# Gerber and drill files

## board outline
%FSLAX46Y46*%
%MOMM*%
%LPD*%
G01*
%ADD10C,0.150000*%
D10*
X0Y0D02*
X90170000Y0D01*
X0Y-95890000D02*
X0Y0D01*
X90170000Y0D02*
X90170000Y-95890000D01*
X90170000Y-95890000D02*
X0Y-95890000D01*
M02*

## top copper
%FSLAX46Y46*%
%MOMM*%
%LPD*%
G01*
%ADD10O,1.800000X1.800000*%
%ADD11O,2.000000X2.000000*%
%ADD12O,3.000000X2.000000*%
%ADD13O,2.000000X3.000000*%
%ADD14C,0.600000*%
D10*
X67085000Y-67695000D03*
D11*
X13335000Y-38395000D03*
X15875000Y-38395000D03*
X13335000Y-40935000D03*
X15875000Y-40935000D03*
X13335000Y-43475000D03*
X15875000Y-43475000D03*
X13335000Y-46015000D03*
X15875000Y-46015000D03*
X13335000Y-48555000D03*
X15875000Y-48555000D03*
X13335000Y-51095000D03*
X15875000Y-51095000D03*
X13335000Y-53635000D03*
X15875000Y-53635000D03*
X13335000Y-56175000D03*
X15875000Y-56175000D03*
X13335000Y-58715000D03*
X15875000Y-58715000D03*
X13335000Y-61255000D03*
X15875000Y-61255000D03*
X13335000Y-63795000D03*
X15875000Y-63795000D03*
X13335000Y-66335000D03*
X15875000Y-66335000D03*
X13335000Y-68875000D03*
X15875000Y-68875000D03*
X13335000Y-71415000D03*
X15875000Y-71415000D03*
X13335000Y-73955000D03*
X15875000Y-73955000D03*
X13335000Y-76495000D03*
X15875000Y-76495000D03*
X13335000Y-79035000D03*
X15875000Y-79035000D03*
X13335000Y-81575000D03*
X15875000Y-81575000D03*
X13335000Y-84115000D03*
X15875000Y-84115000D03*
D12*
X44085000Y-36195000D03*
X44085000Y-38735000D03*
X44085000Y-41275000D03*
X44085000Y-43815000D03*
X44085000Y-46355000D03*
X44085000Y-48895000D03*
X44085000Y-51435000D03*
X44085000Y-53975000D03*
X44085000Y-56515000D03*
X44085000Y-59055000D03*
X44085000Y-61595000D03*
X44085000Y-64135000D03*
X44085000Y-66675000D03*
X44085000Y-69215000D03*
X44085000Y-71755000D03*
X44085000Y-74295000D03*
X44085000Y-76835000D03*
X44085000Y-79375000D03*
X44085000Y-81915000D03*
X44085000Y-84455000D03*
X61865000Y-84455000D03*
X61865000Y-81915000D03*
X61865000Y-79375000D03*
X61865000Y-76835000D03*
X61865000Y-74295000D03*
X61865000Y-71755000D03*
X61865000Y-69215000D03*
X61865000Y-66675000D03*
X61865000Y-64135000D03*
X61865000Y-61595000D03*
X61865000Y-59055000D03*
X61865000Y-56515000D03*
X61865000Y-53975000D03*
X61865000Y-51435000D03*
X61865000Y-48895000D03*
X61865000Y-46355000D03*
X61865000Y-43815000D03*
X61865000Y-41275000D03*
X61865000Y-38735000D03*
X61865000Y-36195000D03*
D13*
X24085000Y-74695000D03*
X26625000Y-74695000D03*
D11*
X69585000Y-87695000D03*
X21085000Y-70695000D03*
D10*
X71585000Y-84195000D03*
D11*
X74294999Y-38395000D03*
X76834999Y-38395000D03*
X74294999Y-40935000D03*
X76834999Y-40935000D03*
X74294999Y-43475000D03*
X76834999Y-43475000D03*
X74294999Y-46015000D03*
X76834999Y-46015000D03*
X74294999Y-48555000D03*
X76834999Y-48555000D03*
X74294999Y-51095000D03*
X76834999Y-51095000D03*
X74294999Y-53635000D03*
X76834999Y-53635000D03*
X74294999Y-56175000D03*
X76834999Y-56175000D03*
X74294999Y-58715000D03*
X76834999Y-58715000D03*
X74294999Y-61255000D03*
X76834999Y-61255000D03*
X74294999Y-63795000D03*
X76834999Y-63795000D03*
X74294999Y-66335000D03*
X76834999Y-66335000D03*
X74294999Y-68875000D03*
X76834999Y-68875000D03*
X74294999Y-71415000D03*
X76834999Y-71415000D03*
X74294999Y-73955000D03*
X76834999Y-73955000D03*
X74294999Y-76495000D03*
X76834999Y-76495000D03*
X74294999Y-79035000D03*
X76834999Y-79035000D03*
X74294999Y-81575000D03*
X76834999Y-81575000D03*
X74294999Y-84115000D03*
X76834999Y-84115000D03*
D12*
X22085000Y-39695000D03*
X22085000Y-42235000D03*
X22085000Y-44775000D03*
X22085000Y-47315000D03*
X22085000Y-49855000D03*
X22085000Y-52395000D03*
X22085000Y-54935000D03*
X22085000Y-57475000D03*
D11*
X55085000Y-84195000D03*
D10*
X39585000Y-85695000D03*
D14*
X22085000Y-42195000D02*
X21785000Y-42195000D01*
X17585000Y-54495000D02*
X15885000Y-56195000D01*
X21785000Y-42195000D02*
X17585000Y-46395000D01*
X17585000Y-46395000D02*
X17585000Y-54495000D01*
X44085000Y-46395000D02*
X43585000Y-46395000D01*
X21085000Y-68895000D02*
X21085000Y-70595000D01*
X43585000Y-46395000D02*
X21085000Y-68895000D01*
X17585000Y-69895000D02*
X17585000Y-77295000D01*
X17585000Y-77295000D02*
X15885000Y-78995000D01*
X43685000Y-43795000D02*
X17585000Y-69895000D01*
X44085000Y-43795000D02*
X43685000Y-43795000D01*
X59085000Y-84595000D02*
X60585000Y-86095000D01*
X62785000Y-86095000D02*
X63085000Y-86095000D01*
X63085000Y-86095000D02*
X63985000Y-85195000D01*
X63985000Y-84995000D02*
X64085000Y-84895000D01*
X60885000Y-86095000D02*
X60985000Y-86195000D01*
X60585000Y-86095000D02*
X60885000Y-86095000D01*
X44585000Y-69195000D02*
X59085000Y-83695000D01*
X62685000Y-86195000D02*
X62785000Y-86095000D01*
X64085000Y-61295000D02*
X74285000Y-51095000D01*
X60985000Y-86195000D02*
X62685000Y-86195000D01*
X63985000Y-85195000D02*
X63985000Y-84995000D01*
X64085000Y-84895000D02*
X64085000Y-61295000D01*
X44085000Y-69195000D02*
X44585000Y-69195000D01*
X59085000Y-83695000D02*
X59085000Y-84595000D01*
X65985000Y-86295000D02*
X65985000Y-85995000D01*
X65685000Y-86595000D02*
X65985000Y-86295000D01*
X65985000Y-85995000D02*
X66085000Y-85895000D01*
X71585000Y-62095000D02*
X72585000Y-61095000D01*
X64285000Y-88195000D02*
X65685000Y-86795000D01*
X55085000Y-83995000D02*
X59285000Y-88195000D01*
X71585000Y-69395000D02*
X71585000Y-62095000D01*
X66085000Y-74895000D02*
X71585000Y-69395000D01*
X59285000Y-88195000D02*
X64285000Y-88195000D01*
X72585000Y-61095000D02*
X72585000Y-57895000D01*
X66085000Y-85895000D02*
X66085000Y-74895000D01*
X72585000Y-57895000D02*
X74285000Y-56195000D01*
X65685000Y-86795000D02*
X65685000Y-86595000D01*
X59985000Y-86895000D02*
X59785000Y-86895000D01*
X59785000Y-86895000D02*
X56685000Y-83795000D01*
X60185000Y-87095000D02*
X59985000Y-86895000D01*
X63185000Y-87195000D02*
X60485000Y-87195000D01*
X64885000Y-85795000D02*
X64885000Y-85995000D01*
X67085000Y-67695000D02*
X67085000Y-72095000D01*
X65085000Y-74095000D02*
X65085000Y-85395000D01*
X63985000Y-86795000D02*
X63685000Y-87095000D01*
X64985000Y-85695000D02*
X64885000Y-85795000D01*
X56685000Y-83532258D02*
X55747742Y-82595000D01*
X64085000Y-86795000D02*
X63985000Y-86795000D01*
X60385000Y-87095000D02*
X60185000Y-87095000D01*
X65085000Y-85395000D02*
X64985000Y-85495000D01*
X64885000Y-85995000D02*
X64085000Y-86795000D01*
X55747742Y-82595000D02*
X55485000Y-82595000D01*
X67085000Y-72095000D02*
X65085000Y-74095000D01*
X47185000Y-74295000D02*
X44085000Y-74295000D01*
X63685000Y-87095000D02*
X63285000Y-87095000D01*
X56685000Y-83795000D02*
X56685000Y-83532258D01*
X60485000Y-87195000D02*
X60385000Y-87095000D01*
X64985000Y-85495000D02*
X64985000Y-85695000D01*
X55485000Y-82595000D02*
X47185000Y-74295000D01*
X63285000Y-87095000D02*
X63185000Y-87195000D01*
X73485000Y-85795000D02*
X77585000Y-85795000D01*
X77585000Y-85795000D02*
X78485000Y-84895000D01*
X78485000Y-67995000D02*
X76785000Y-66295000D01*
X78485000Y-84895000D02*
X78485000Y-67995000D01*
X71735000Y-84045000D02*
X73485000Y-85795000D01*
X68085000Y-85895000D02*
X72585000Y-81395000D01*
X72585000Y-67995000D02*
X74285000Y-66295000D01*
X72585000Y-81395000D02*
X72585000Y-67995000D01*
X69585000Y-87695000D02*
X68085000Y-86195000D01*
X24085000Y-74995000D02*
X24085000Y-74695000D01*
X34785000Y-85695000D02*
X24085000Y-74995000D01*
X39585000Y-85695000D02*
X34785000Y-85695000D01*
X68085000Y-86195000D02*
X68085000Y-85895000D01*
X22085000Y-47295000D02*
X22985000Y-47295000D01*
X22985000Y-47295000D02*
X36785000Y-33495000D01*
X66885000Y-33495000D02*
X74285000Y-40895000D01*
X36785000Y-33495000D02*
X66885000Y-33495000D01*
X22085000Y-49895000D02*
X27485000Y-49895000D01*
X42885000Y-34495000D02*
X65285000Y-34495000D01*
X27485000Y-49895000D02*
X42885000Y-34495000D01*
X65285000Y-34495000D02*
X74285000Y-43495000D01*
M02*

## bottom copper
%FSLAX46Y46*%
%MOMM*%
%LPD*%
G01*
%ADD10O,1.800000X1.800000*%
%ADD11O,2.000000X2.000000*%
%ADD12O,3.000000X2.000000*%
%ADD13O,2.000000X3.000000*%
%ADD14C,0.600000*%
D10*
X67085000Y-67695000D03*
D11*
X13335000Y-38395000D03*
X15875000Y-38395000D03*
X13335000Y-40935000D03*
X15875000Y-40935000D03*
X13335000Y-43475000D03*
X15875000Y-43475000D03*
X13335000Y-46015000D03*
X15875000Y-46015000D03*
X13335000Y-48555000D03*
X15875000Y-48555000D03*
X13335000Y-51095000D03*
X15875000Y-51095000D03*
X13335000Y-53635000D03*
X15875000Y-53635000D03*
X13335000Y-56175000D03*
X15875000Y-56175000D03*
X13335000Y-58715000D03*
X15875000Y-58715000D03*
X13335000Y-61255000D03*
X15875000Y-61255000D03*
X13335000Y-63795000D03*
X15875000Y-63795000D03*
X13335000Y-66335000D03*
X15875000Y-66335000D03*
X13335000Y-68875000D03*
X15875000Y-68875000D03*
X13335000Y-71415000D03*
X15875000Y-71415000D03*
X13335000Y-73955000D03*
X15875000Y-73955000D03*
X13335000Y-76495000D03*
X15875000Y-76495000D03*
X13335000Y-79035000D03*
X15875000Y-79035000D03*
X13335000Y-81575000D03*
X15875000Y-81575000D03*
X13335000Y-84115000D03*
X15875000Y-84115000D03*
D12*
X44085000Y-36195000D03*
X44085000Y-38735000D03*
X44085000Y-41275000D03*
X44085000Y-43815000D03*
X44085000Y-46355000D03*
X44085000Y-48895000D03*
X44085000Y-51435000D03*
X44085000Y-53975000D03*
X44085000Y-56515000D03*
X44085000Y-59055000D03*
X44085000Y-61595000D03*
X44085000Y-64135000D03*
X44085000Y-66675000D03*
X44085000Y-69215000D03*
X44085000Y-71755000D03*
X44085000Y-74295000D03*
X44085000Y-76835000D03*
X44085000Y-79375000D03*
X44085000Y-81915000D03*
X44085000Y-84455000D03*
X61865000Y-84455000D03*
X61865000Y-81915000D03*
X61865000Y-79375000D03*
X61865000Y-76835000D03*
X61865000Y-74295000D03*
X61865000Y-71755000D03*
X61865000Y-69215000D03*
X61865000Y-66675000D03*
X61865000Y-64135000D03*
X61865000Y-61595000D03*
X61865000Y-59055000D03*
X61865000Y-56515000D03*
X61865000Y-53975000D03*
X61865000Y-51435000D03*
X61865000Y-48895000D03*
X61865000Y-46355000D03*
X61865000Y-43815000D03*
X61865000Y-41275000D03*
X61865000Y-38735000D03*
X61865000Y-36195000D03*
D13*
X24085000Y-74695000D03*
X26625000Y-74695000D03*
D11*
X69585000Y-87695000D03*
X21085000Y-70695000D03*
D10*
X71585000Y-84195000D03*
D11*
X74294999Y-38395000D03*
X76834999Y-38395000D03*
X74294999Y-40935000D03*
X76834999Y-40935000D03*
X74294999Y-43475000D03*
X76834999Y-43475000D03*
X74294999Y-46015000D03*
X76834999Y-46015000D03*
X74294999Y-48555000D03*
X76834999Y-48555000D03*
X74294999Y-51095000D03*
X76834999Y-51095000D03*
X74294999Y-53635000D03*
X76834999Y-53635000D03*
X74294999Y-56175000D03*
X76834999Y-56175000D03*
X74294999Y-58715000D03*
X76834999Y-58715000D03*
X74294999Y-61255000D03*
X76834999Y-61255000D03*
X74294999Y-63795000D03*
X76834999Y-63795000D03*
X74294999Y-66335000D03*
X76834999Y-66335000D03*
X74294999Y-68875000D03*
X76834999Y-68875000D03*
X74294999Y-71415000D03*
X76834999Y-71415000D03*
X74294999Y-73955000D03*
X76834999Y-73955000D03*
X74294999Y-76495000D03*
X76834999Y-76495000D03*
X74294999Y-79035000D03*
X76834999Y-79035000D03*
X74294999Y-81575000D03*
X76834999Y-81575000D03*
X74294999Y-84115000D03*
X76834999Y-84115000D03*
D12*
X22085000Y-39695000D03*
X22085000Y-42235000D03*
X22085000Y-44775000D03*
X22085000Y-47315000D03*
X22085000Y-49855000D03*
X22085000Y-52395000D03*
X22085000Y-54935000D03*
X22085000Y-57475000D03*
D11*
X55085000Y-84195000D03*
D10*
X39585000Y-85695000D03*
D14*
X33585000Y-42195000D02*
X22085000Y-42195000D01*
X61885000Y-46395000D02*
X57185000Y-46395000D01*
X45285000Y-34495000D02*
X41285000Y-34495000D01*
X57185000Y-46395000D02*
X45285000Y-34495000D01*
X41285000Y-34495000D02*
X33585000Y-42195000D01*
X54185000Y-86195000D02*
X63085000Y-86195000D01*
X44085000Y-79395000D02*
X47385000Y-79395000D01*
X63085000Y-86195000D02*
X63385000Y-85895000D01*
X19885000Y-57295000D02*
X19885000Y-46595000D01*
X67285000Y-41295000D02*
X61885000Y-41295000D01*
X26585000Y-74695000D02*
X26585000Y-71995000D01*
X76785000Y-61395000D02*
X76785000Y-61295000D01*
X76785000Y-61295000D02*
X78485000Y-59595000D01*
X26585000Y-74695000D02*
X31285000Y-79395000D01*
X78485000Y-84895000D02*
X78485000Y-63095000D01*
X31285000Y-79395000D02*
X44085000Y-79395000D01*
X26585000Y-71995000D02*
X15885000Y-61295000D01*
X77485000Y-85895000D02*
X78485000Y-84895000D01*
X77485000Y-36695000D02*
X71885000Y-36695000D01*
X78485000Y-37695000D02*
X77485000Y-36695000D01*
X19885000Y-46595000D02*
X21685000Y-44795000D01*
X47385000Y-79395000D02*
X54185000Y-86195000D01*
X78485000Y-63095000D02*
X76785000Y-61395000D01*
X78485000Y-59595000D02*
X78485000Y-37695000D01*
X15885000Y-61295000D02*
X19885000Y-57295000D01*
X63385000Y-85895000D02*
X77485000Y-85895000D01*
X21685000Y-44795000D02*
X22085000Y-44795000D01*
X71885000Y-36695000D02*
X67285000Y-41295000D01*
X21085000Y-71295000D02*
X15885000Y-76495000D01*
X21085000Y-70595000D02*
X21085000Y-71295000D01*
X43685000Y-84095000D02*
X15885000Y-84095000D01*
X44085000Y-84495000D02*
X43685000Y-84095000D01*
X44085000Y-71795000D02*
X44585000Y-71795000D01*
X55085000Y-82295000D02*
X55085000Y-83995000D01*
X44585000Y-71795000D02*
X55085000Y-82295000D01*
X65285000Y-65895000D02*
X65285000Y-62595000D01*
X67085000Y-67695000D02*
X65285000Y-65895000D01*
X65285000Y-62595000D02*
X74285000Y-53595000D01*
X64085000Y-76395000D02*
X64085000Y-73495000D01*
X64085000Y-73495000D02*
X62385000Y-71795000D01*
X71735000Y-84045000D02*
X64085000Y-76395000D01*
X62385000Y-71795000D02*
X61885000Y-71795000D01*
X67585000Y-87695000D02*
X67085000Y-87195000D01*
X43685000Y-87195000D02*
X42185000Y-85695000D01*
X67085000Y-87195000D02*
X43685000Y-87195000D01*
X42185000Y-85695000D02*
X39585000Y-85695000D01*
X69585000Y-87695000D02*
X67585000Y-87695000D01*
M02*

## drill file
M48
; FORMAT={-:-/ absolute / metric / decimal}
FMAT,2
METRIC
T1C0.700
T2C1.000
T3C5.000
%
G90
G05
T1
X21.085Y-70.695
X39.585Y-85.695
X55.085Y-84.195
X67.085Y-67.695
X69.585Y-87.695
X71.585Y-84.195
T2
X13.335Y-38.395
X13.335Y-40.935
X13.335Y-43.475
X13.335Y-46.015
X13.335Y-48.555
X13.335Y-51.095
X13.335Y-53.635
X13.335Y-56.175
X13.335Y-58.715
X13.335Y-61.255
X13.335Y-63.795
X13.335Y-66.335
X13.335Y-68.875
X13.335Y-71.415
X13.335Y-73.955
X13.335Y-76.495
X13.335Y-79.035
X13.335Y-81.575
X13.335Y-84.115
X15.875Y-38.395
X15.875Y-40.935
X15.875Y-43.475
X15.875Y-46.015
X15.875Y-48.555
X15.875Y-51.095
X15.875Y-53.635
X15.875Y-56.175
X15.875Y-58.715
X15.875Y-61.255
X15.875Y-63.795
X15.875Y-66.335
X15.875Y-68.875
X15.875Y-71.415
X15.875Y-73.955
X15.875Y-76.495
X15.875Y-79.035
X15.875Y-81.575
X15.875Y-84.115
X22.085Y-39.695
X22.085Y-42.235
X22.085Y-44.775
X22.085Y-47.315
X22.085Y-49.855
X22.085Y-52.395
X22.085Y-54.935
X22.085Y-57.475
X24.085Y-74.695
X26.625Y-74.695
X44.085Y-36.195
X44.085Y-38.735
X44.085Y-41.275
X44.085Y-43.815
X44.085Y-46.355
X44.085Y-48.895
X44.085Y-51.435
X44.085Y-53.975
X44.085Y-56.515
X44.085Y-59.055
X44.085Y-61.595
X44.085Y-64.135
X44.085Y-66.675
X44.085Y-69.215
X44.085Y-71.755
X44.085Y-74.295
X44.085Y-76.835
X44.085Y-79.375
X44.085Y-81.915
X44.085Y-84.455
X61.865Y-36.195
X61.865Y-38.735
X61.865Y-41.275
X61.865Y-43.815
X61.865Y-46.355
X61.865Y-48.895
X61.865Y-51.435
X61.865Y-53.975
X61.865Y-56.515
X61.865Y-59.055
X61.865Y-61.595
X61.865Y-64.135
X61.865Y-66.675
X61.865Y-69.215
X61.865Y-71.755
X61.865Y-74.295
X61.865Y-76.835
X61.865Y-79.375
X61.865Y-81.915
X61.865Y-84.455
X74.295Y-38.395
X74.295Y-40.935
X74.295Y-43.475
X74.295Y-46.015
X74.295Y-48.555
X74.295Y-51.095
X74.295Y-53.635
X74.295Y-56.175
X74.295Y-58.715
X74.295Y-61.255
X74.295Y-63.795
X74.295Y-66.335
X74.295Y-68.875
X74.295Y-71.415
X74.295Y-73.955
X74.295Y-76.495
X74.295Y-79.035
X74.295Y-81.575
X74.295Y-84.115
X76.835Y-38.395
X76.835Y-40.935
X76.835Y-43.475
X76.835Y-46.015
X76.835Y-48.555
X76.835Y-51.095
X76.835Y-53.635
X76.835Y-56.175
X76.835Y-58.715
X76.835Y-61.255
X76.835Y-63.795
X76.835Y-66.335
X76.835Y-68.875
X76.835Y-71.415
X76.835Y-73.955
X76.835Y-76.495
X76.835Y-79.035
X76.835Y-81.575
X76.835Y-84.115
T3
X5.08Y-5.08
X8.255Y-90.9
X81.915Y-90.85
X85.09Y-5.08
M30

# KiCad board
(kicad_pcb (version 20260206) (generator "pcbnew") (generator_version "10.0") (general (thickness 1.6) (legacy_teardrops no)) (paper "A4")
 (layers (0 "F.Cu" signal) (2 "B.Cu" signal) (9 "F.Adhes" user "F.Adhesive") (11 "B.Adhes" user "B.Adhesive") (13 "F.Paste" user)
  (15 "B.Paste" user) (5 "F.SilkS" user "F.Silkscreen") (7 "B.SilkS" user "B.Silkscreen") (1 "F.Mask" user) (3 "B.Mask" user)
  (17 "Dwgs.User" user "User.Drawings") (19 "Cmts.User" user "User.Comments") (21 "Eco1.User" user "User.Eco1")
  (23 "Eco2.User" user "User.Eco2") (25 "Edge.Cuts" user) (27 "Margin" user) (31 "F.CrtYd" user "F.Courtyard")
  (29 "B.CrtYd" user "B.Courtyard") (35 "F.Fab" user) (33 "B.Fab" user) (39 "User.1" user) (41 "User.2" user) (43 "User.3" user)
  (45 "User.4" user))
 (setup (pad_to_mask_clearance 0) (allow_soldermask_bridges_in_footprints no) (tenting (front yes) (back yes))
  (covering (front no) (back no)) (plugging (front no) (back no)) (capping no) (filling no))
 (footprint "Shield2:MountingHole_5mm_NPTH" (layer "F.Cu") (at 5.08 5.08)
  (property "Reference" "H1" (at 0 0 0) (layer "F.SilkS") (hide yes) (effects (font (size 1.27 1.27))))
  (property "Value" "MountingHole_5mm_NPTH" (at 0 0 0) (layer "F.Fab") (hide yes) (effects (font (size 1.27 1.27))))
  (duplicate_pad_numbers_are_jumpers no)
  (pad "" np_thru_hole circle (at 0 0) (size 5 5) (drill 5) (layers "*.Cu")))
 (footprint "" (layer "F.Cu") (at 67.085 67.695)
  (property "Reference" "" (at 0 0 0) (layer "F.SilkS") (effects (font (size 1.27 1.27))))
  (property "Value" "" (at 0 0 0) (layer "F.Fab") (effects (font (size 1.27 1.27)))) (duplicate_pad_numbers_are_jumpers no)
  (pad "2" thru_hole oval (at 0 0) (size 1.8 1.8) (drill 0.7) (layers "*.Cu") (remove_unused_layers no)))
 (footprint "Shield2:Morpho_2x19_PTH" (layer "F.Cu") (at 13.335 38.395)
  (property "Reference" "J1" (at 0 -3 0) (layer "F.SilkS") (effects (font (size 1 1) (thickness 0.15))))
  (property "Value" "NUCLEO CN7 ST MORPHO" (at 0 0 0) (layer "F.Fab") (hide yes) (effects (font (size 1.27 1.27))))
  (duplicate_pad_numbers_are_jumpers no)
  (pad "1" thru_hole oval (at 0 0) (size 2 2) (drill 1) (layers "*.Cu") (remove_unused_layers no) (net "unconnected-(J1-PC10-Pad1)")
   (thermal_bridge_angle 45))
  (pad "2" thru_hole oval (at 2.54 0) (size 2 2) (drill 1) (layers "*.Cu") (remove_unused_layers no) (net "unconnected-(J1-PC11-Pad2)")
   (thermal_bridge_angle 45))
  (pad "3" thru_hole oval (at 0 2.54) (size 2 2) (drill 1) (layers "*.Cu") (remove_unused_layers no) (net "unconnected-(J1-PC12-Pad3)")
   (thermal_bridge_angle 45))
  (pad "4" thru_hole oval (at 2.54 2.54) (size 2 2) (drill 1) (layers "*.Cu") (remove_unused_layers no) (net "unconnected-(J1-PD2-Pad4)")
   (thermal_bridge_angle 45))
  (pad "5" thru_hole oval (at 0 5.08) (size 2 2) (drill 1) (layers "*.Cu") (remove_unused_layers no) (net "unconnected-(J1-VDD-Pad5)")
   (thermal_bridge_angle 45))
  (pad "6" thru_hole oval (at 2.54 5.08) (size 2 2) (drill 1) (layers "*.Cu") (remove_unused_layers no) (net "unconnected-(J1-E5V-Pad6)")
   (thermal_bridge_angle 45))
  (pad "7" thru_hole oval (at 0 7.62) (size 2 2) (drill 1) (layers "*.Cu") (remove_unused_layers no) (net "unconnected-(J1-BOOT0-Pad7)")
   (thermal_bridge_angle 45))
  (pad "8" thru_hole oval (at 2.54 7.62) (size 2 2) (drill 1) (layers "*.Cu") (remove_unused_layers no) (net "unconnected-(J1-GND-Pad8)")
   (thermal_bridge_angle 45))
  (pad "9" thru_hole oval (at 0 10.16) (size 2 2) (drill 1) (layers "*.Cu") (remove_unused_layers no) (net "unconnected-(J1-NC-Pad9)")
   (thermal_bridge_angle 45))
  (pad "10" thru_hole oval (at 2.54 10.16) (size 2 2) (drill 1) (layers "*.Cu") (remove_unused_layers no) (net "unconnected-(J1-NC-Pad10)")
   (thermal_bridge_angle 45))
  (pad "11" thru_hole oval (at 0 12.7) (size 2 2) (drill 1) (layers "*.Cu") (remove_unused_layers no) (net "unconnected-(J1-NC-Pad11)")
   (thermal_bridge_angle 45))
  (pad "12" thru_hole oval (at 2.54 12.7) (size 2 2) (drill 1) (layers "*.Cu") (remove_unused_layers no)
   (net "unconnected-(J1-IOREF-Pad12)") (thermal_bridge_angle 45))
  (pad "13" thru_hole oval (at 0 15.24) (size 2 2) (drill 1) (layers "*.Cu") (remove_unused_layers no) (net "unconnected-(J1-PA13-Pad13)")
   (thermal_bridge_angle 45))
  (pad "14" thru_hole oval (at 2.54 15.24) (size 2 2) (drill 1) (layers "*.Cu") (remove_unused_layers no)
   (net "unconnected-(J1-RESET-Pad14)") (thermal_bridge_angle 45))
  (pad "15" thru_hole oval (at 0 17.78) (size 2 2) (drill 1) (layers "*.Cu") (remove_unused_layers no) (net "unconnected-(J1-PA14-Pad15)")
   (thermal_bridge_angle 45))
  (pad "16" thru_hole oval (at 2.54 17.78) (size 2 2) (drill 1) (layers "*.Cu") (remove_unused_layers no) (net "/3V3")
   (thermal_bridge_angle 45))
  (pad "17" thru_hole oval (at 0 20.32) (size 2 2) (drill 1) (layers "*.Cu") (remove_unused_layers no) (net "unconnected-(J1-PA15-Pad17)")
   (thermal_bridge_angle 45))
  (pad "18" thru_hole oval (at 2.54 20.32) (size 2 2) (drill 1) (layers "*.Cu") (remove_unused_layers no) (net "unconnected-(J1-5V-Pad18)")
   (thermal_bridge_angle 45))
  (pad "19" thru_hole oval (at 0 22.86) (size 2 2) (drill 1) (layers "*.Cu") (remove_unused_layers no) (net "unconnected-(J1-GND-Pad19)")
   (thermal_bridge_angle 45))
  (pad "20" thru_hole oval (at 2.54 22.86) (size 2 2) (drill 1) (layers "*.Cu") (remove_unused_layers no) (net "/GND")
   (thermal_bridge_angle 45))
  (pad "21" thru_hole oval (at 0 25.4) (size 2 2) (drill 1) (layers "*.Cu") (remove_unused_layers no) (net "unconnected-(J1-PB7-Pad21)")
   (thermal_bridge_angle 45))
  (pad "22" thru_hole oval (at 2.54 25.4) (size 2 2) (drill 1) (layers "*.Cu") (remove_unused_layers no) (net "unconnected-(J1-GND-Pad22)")
   (thermal_bridge_angle 45))
  (pad "23" thru_hole oval (at 0 27.94) (size 2 2) (drill 1) (layers "*.Cu") (remove_unused_layers no) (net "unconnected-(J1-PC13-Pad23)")
   (thermal_bridge_angle 45))
  (pad "24" thru_hole oval (at 2.54 27.94) (size 2 2) (drill 1) (layers "*.Cu") (remove_unused_layers no) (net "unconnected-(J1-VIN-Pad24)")
   (thermal_bridge_angle 45))
  (pad "25" thru_hole oval (at 0 30.48) (size 2 2) (drill 1) (layers "*.Cu") (remove_unused_layers no) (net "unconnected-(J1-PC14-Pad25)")
   (thermal_bridge_angle 45))
  (pad "26" thru_hole oval (at 2.54 30.48) (size 2 2) (drill 1) (layers "*.Cu") (remove_unused_layers no) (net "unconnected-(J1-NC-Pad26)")
   (thermal_bridge_angle 45))
  (pad "27" thru_hole oval (at 0 33.02) (size 2 2) (drill 1) (layers "*.Cu") (remove_unused_layers no) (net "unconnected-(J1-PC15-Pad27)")
   (thermal_bridge_angle 45))
  (pad "28" thru_hole oval (at 2.54 33.02) (size 2 2) (drill 1) (layers "*.Cu") (remove_unused_layers no) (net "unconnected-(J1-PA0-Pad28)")
   (thermal_bridge_angle 45))
  (pad "29" thru_hole oval (at 0 35.56) (size 2 2) (drill 1) (layers "*.Cu") (remove_unused_layers no) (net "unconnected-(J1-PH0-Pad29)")
   (thermal_bridge_angle 45))
  (pad "30" thru_hole oval (at 2.54 35.56) (size 2 2) (drill 1) (layers "*.Cu") (remove_unused_layers no) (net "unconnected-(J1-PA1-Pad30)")
   (thermal_bridge_angle 45))
  (pad "31" thru_hole oval (at 0 38.1) (size 2 2) (drill 1) (layers "*.Cu") (remove_unused_layers no) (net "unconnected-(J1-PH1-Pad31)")
   (thermal_bridge_angle 45))
  (pad "32" thru_hole oval (at 2.54 38.1) (size 2 2) (drill 1) (layers "*.Cu") (remove_unused_layers no) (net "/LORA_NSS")
   (thermal_bridge_angle 45))
  (pad "33" thru_hole oval (at 0 40.64) (size 2 2) (drill 1) (layers "*.Cu") (remove_unused_layers no) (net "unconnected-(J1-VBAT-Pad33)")
   (thermal_bridge_angle 45))
  (pad "34" thru_hole oval (at 2.54 40.64) (size 2 2) (drill 1) (layers "*.Cu") (remove_unused_layers no) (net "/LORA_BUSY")
   (thermal_bridge_angle 45))
  (pad "35" thru_hole oval (at 0 43.18) (size 2 2) (drill 1) (layers "*.Cu") (remove_unused_layers no) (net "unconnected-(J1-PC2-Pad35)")
   (thermal_bridge_angle 45))
  (pad "36" thru_hole oval (at 2.54 43.18) (size 2 2) (drill 1) (layers "*.Cu") (remove_unused_layers no)
   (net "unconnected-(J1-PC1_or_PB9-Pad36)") (thermal_bridge_angle 45))
  (pad "37" thru_hole oval (at 0 45.72) (size 2 2) (drill 1) (layers "*.Cu") (remove_unused_layers no) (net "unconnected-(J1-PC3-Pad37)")
   (thermal_bridge_angle 45))
  (pad "38" thru_hole oval (at 2.54 45.72) (size 2 2) (drill 1) (layers "*.Cu") (remove_unused_layers no) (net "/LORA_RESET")
   (thermal_bridge_angle 45)))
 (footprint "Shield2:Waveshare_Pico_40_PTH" (layer "F.Cu") (at 44.085 36.195)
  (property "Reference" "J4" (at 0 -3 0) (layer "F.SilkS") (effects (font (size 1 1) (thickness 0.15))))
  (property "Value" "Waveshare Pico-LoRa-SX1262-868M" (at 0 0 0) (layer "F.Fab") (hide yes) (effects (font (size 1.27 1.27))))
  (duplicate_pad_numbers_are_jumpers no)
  (pad "1" thru_hole oval (at 0 0) (size 3 2) (drill 1) (layers "*.Cu") (remove_unused_layers no) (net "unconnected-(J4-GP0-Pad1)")
   (thermal_bridge_angle 45))
  (pad "2" thru_hole oval (at 0 2.54) (size 3 2) (drill 1) (layers "*.Cu") (remove_unused_layers no) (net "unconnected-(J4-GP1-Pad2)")
   (thermal_bridge_angle 45))
  (pad "3" thru_hole oval (at 0 5.08) (size 3 2) (drill 1) (layers "*.Cu") (remove_unused_layers no) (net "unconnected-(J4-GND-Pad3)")
   (thermal_bridge_angle 45))
  (pad "4" thru_hole oval (at 0 7.62) (size 3 2) (drill 1) (layers "*.Cu") (remove_unused_layers no) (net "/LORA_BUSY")
   (thermal_bridge_angle 45))
  (pad "5" thru_hole oval (at 0 10.16) (size 3 2) (drill 1) (layers "*.Cu") (remove_unused_layers no) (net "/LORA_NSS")
   (thermal_bridge_angle 45))
  (pad "6" thru_hole oval (at 0 12.7) (size 3 2) (drill 1) (layers "*.Cu") (remove_unused_layers no) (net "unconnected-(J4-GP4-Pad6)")
   (thermal_bridge_angle 45))
  (pad "7" thru_hole oval (at 0 15.24) (size 3 2) (drill 1) (layers "*.Cu") (remove_unused_layers no) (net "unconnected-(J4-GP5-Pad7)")
   (thermal_bridge_angle 45))
  (pad "8" thru_hole oval (at 0 17.78) (size 3 2) (drill 1) (layers "*.Cu") (remove_unused_layers no) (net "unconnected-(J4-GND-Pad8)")
   (thermal_bridge_angle 45))
  (pad "9" thru_hole oval (at 0 20.32) (size 3 2) (drill 1) (layers "*.Cu") (remove_unused_layers no) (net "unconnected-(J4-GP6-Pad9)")
   (thermal_bridge_angle 45))
  (pad "10" thru_hole oval (at 0 22.86) (size 3 2) (drill 1) (layers "*.Cu") (remove_unused_layers no) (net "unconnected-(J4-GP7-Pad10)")
   (thermal_bridge_angle 45))
  (pad "11" thru_hole oval (at 0 25.4) (size 3 2) (drill 1) (layers "*.Cu") (remove_unused_layers no) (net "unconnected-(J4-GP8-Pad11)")
   (thermal_bridge_angle 45))
  (pad "12" thru_hole oval (at 0 27.94) (size 3 2) (drill 1) (layers "*.Cu") (remove_unused_layers no) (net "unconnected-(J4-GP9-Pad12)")
   (thermal_bridge_angle 45))
  (pad "13" thru_hole oval (at 0 30.48) (size 3 2) (drill 1) (layers "*.Cu") (remove_unused_layers no) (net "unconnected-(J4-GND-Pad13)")
   (thermal_bridge_angle 45))
  (pad "14" thru_hole oval (at 0 33.02) (size 3 2) (drill 1) (layers "*.Cu") (remove_unused_layers no) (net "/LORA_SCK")
   (thermal_bridge_angle 45))
  (pad "15" thru_hole oval (at 0 35.56) (size 3 2) (drill 1) (layers "*.Cu") (remove_unused_layers no) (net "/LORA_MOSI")
   (thermal_bridge_angle 45))
  (pad "16" thru_hole oval (at 0 38.1) (size 3 2) (drill 1) (layers "*.Cu") (remove_unused_layers no) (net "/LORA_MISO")
   (thermal_bridge_angle 45))
  (pad "17" thru_hole oval (at 0 40.64) (size 3 2) (drill 1) (layers "*.Cu") (remove_unused_layers no) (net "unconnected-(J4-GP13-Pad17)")
   (thermal_bridge_angle 45))
  (pad "18" thru_hole oval (at 0 43.18) (size 3 2) (drill 1) (layers "*.Cu") (remove_unused_layers no) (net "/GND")
   (thermal_bridge_angle 45))
  (pad "19" thru_hole oval (at 0 45.72) (size 3 2) (drill 1) (layers "*.Cu") (remove_unused_layers no) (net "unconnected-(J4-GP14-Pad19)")
   (thermal_bridge_angle 45))
  (pad "20" thru_hole oval (at 0 48.26) (size 3 2) (drill 1) (layers "*.Cu") (remove_unused_layers no) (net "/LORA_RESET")
   (thermal_bridge_angle 45))
  (pad "21" thru_hole oval (at 17.78 48.26) (size 3 2) (drill 1) (layers "*.Cu") (remove_unused_layers no)
   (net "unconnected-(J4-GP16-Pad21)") (thermal_bridge_angle 45))
  (pad "22" thru_hole oval (at 17.78 45.72) (size 3 2) (drill 1) (layers "*.Cu") (remove_unused_layers no)
   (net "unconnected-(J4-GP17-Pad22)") (thermal_bridge_angle 45))
  (pad "23" thru_hole oval (at 17.78 43.18) (size 3 2) (drill 1) (layers "*.Cu") (remove_unused_layers no)
   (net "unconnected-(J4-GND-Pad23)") (thermal_bridge_angle 45))
  (pad "24" thru_hole oval (at 17.78 40.64) (size 3 2) (drill 1) (layers "*.Cu") (remove_unused_layers no)
   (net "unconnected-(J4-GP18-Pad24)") (thermal_bridge_angle 45))
  (pad "25" thru_hole oval (at 17.78 38.1) (size 3 2) (drill 1) (layers "*.Cu") (remove_unused_layers no)
   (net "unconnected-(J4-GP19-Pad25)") (thermal_bridge_angle 45))
  (pad "26" thru_hole oval (at 17.78 35.56) (size 3 2) (drill 1) (layers "*.Cu") (remove_unused_layers no) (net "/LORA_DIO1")
   (thermal_bridge_angle 45))
  (pad "27" thru_hole oval (at 17.78 33.02) (size 3 2) (drill 1) (layers "*.Cu") (remove_unused_layers no)
   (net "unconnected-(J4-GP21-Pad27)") (thermal_bridge_angle 45))
  (pad "28" thru_hole oval (at 17.78 30.48) (size 3 2) (drill 1) (layers "*.Cu") (remove_unused_layers no)
   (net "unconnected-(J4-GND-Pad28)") (thermal_bridge_angle 45))
  (pad "29" thru_hole oval (at 17.78 27.94) (size 3 2) (drill 1) (layers "*.Cu") (remove_unused_layers no)
   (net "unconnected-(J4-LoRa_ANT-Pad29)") (thermal_bridge_angle 45))
  (pad "30" thru_hole oval (at 17.78 25.4) (size 3 2) (drill 1) (layers "*.Cu") (remove_unused_layers no) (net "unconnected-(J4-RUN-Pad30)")
   (thermal_bridge_angle 45))
  (pad "31" thru_hole oval (at 17.78 22.86) (size 3 2) (drill 1) (layers "*.Cu") (remove_unused_layers no)
   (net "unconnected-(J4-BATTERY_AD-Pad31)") (thermal_bridge_angle 45))
  (pad "32" thru_hole oval (at 17.78 20.32) (size 3 2) (drill 1) (layers "*.Cu") (remove_unused_layers no)
   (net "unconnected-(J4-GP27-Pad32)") (thermal_bridge_angle 45))
  (pad "33" thru_hole oval (at 17.78 17.78) (size 3 2) (drill 1) (layers "*.Cu") (remove_unused_layers no)
   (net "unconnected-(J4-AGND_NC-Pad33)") (thermal_bridge_angle 45))
  (pad "34" thru_hole oval (at 17.78 15.24) (size 3 2) (drill 1) (layers "*.Cu") (remove_unused_layers no)
   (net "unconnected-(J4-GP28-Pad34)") (thermal_bridge_angle 45))
  (pad "35" thru_hole oval (at 17.78 12.7) (size 3 2) (drill 1) (layers "*.Cu") (remove_unused_layers no)
   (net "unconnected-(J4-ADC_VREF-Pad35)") (thermal_bridge_angle 45))
  (pad "36" thru_hole oval (at 17.78 10.16) (size 3 2) (drill 1) (layers "*.Cu") (remove_unused_layers no) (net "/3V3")
   (thermal_bridge_angle 45))
  (pad "37" thru_hole oval (at 17.78 7.62) (size 3 2) (drill 1) (layers "*.Cu") (remove_unused_layers no)
   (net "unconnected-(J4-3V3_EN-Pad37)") (thermal_bridge_angle 45))
  (pad "38" thru_hole oval (at 17.78 5.08) (size 3 2) (drill 1) (layers "*.Cu") (remove_unused_layers no) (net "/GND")
   (thermal_bridge_angle 45))
  (pad "39" thru_hole oval (at 17.78 2.54) (size 3 2) (drill 1) (layers "*.Cu") (remove_unused_layers no)
   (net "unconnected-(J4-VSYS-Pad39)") (thermal_bridge_angle 45))
  (pad "40" thru_hole oval (at 17.78 0) (size 3 2) (drill 1) (layers "*.Cu") (remove_unused_layers no) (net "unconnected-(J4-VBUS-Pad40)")
   (thermal_bridge_angle 45)))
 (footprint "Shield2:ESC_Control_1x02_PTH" (layer "F.Cu") (at 24.085 74.695)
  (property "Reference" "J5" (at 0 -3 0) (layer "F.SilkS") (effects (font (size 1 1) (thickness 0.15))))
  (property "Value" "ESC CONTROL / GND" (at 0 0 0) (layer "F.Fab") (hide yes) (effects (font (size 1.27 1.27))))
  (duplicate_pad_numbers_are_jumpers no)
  (pad "1" thru_hole oval (at 0 0) (size 2 3) (drill 1) (layers "*.Cu") (remove_unused_layers no) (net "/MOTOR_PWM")
   (thermal_bridge_angle 45))
  (pad "2" thru_hole oval (at 2.54 0) (size 2 3) (drill 1) (layers "*.Cu") (remove_unused_layers no) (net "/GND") (thermal_bridge_angle 45)))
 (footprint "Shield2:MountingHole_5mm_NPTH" (layer "F.Cu") (at 8.255 90.9)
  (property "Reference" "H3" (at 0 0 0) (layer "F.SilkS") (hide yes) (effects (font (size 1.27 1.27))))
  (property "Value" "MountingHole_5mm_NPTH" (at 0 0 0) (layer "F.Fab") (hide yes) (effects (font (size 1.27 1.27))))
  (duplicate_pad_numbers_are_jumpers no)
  (pad "" np_thru_hole circle (at 0 0) (size 5 5) (drill 5) (layers "*.Cu")))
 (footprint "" (layer "F.Cu") (at 69.585 87.695)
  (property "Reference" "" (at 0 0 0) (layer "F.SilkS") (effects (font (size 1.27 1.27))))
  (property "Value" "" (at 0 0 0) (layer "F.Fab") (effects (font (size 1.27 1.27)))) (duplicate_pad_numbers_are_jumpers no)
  (pad "2" thru_hole oval (at 0 0) (size 2 2) (drill 0.7) (layers "*.Cu") (remove_unused_layers no)))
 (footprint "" (layer "F.Cu") (at 21.085 70.695)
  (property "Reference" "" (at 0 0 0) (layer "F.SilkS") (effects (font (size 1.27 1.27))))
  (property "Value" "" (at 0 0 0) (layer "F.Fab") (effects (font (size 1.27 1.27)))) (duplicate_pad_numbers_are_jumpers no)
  (pad "2" thru_hole oval (at 0 0) (size 2 2) (drill 0.7) (layers "*.Cu") (remove_unused_layers no)))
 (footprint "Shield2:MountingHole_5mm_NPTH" (layer "F.Cu") (at 85.09 5.08)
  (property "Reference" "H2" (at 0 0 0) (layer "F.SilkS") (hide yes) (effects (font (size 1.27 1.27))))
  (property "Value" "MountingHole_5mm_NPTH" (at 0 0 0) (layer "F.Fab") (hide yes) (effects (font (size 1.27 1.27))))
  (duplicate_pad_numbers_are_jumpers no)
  (pad "" np_thru_hole circle (at 0 0) (size 5 5) (drill 5) (layers "*.Cu")))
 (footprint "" (layer "F.Cu") (at 71.585 84.195)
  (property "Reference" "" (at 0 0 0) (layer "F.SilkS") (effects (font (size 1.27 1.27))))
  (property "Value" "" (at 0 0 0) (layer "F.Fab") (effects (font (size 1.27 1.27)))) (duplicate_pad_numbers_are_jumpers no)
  (pad "2" thru_hole oval (at 0 0) (size 1.8 1.8) (drill 0.7) (layers "*.Cu") (remove_unused_layers no)))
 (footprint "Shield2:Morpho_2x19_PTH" (layer "F.Cu") (at 74.294999 38.395)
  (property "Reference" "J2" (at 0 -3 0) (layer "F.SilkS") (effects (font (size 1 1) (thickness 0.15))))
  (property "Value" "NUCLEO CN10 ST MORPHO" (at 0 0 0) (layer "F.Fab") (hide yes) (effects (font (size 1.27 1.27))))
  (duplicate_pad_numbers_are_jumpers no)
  (pad "1" thru_hole oval (at 0 0) (size 2 2) (drill 1) (layers "*.Cu") (remove_unused_layers no) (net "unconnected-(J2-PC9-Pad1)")
   (thermal_bridge_angle 45))
  (pad "2" thru_hole oval (at 2.54 0) (size 2 2) (drill 1) (layers "*.Cu") (remove_unused_layers no) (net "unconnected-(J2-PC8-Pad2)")
   (thermal_bridge_angle 45))
  (pad "3" thru_hole oval (at 0 2.54) (size 2 2) (drill 1) (layers "*.Cu") (remove_unused_layers no) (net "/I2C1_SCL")
   (thermal_bridge_angle 45))
  (pad "4" thru_hole oval (at 2.54 2.54) (size 2 2) (drill 1) (layers "*.Cu") (remove_unused_layers no) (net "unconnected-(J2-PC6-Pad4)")
   (thermal_bridge_angle 45))
  (pad "5" thru_hole oval (at 0 5.08) (size 2 2) (drill 1) (layers "*.Cu") (remove_unused_layers no) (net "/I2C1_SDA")
   (thermal_bridge_angle 45))
  (pad "6" thru_hole oval (at 2.54 5.08) (size 2 2) (drill 1) (layers "*.Cu") (remove_unused_layers no) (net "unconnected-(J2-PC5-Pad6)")
   (thermal_bridge_angle 45))
  (pad "7" thru_hole oval (at 0 7.62) (size 2 2) (drill 1) (layers "*.Cu") (remove_unused_layers no) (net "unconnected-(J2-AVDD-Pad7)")
   (thermal_bridge_angle 45))
  (pad "8" thru_hole oval (at 2.54 7.62) (size 2 2) (drill 1) (layers "*.Cu") (remove_unused_layers no) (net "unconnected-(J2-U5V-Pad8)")
   (thermal_bridge_angle 45))
  (pad "9" thru_hole oval (at 0 10.16) (size 2 2) (drill 1) (layers "*.Cu") (remove_unused_layers no) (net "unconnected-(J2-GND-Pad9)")
   (thermal_bridge_angle 45))
  (pad "10" thru_hole oval (at 2.54 10.16) (size 2 2) (drill 1) (layers "*.Cu") (remove_unused_layers no) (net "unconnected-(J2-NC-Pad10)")
   (thermal_bridge_angle 45))
  (pad "11" thru_hole oval (at 0 12.7) (size 2 2) (drill 1) (layers "*.Cu") (remove_unused_layers no) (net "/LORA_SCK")
   (thermal_bridge_angle 45))
  (pad "12" thru_hole oval (at 2.54 12.7) (size 2 2) (drill 1) (layers "*.Cu") (remove_unused_layers no) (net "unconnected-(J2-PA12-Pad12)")
   (thermal_bridge_angle 45))
  (pad "13" thru_hole oval (at 0 15.24) (size 2 2) (drill 1) (layers "*.Cu") (remove_unused_layers no) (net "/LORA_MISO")
   (thermal_bridge_angle 45))
  (pad "14" thru_hole oval (at 2.54 15.24) (size 2 2) (drill 1) (layers "*.Cu") (remove_unused_layers no)
   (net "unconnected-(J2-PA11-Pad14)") (thermal_bridge_angle 45))
  (pad "15" thru_hole oval (at 0 17.78) (size 2 2) (drill 1) (layers "*.Cu") (remove_unused_layers no) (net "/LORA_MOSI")
   (thermal_bridge_angle 45))
  (pad "16" thru_hole oval (at 2.54 17.78) (size 2 2) (drill 1) (layers "*.Cu") (remove_unused_layers no)
   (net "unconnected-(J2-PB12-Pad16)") (thermal_bridge_angle 45))
  (pad "17" thru_hole oval (at 0 20.32) (size 2 2) (drill 1) (layers "*.Cu") (remove_unused_layers no) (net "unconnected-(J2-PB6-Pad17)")
   (thermal_bridge_angle 45))
  (pad "18" thru_hole oval (at 2.54 20.32) (size 2 2) (drill 1) (layers "*.Cu") (remove_unused_layers no)
   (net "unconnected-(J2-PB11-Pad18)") (thermal_bridge_angle 45))
  (pad "19" thru_hole oval (at 0 22.86) (size 2 2) (drill 1) (layers "*.Cu") (remove_unused_layers no) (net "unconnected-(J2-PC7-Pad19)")
   (thermal_bridge_angle 45))
  (pad "20" thru_hole oval (at 2.54 22.86) (size 2 2) (drill 1) (layers "*.Cu") (remove_unused_layers no) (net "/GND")
   (thermal_bridge_angle 45))
  (pad "21" thru_hole oval (at 0 25.4) (size 2 2) (drill 1) (layers "*.Cu") (remove_unused_layers no) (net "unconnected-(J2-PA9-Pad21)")
   (thermal_bridge_angle 45))
  (pad "22" thru_hole oval (at 2.54 25.4) (size 2 2) (drill 1) (layers "*.Cu") (remove_unused_layers no) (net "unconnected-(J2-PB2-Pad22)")
   (thermal_bridge_angle 45))
  (pad "23" thru_hole oval (at 0 27.94) (size 2 2) (drill 1) (layers "*.Cu") (remove_unused_layers no) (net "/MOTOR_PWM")
   (thermal_bridge_angle 45))
  (pad "24" thru_hole oval (at 2.54 27.94) (size 2 2) (drill 1) (layers "*.Cu") (remove_unused_layers no) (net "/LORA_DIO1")
   (thermal_bridge_angle 45))
  (pad "25" thru_hole oval (at 0 30.48) (size 2 2) (drill 1) (layers "*.Cu") (remove_unused_layers no) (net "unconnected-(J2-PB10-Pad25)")
   (thermal_bridge_angle 45))
  (pad "26" thru_hole oval (at 2.54 30.48) (size 2 2) (drill 1) (layers "*.Cu") (remove_unused_layers no)
   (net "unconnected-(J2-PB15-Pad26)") (thermal_bridge_angle 45))
  (pad "27" thru_hole oval (at 0 33.02) (size 2 2) (drill 1) (layers "*.Cu") (remove_unused_layers no) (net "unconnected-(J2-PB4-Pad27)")
   (thermal_bridge_angle 45))
  (pad "28" thru_hole oval (at 2.54 33.02) (size 2 2) (drill 1) (layers "*.Cu") (remove_unused_layers no)
   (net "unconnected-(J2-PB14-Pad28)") (thermal_bridge_angle 45))
  (pad "29" thru_hole oval (at 0 35.56) (size 2 2) (drill 1) (layers "*.Cu") (remove_unused_layers no) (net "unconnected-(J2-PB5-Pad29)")
   (thermal_bridge_angle 45))
  (pad "30" thru_hole oval (at 2.54 35.56) (size 2 2) (drill 1) (layers "*.Cu") (remove_unused_layers no)
   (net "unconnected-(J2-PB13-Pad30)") (thermal_bridge_angle 45))
  (pad "31" thru_hole oval (at 0 38.1) (size 2 2) (drill 1) (layers "*.Cu") (remove_unused_layers no) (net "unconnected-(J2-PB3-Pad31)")
   (thermal_bridge_angle 45))
  (pad "32" thru_hole oval (at 2.54 38.1) (size 2 2) (drill 1) (layers "*.Cu") (remove_unused_layers no) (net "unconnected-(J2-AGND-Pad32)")
   (thermal_bridge_angle 45))
  (pad "33" thru_hole oval (at 0 40.64) (size 2 2) (drill 1) (layers "*.Cu") (remove_unused_layers no) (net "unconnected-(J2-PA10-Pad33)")
   (thermal_bridge_angle 45))
  (pad "34" thru_hole oval (at 2.54 40.64) (size 2 2) (drill 1) (layers "*.Cu") (remove_unused_layers no) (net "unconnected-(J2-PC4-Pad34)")
   (thermal_bridge_angle 45))
  (pad "35" thru_hole oval (at 0 43.18) (size 2 2) (drill 1) (layers "*.Cu") (remove_unused_layers no) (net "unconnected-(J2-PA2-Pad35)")
   (thermal_bridge_angle 45))
  (pad "36" thru_hole oval (at 2.54 43.18) (size 2 2) (drill 1) (layers "*.Cu") (remove_unused_layers no) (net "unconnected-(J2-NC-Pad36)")
   (thermal_bridge_angle 45))
  (pad "37" thru_hole oval (at 0 45.72) (size 2 2) (drill 1) (layers "*.Cu") (remove_unused_layers no) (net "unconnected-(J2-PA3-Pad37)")
   (thermal_bridge_angle 45))
  (pad "38" thru_hole oval (at 2.54 45.72) (size 2 2) (drill 1) (layers "*.Cu") (remove_unused_layers no) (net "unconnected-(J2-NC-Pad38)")
   (thermal_bridge_angle 45)))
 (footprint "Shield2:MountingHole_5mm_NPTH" (layer "F.Cu") (at 81.915 90.85)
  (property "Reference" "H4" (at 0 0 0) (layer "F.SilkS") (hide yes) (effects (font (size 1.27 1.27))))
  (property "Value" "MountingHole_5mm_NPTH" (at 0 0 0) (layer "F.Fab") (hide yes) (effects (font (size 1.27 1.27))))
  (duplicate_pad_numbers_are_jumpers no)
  (pad "" np_thru_hole circle (at 0 0) (size 5 5) (drill 5) (layers "*.Cu")))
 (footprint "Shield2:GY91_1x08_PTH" (layer "F.Cu") (at 22.085 39.695)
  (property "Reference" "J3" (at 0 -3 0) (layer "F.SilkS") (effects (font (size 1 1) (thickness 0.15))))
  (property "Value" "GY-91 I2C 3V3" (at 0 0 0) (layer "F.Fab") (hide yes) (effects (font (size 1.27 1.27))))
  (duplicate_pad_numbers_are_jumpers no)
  (pad "1" thru_hole oval (at 0 0) (size 3 2) (drill 1) (layers "*.Cu") (remove_unused_layers no) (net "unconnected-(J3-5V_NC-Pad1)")
   (thermal_bridge_angle 45))
  (pad "2" thru_hole oval (at 0 2.54) (size 3 2) (drill 1) (layers "*.Cu") (remove_unused_layers no) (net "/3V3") (thermal_bridge_angle 45))
  (pad "3" thru_hole oval (at 0 5.08) (size 3 2) (drill 1) (layers "*.Cu") (remove_unused_layers no) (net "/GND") (thermal_bridge_angle 45))
  (pad "4" thru_hole oval (at 0 7.62) (size 3 2) (drill 1) (layers "*.Cu") (remove_unused_layers no) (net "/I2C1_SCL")
   (thermal_bridge_angle 45))
  (pad "5" thru_hole oval (at 0 10.16) (size 3 2) (drill 1) (layers "*.Cu") (remove_unused_layers no) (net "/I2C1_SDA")
   (thermal_bridge_angle 45))
  (pad "6" thru_hole oval (at 0 12.7) (size 3 2) (drill 1) (layers "*.Cu") (remove_unused_layers no) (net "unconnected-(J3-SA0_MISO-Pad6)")
   (thermal_bridge_angle 45))
  (pad "7" thru_hole oval (at 0 15.24) (size 3 2) (drill 1) (layers "*.Cu") (remove_unused_layers no) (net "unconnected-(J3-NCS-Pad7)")
   (thermal_bridge_angle 45))
  (pad "8" thru_hole oval (at 0 17.78) (size 3 2) (drill 1) (layers "*.Cu") (remove_unused_layers no) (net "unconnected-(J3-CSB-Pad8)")
   (thermal_bridge_angle 45)))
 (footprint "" (layer "F.Cu") (at 55.085 84.195)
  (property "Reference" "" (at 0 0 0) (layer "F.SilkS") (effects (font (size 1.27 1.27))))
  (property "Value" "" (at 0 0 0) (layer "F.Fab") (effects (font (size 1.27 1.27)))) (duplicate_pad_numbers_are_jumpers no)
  (pad "2" thru_hole oval (at 0 0) (size 2 2) (drill 0.7) (layers "*.Cu") (remove_unused_layers no)))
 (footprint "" (layer "F.Cu") (at 39.585 85.695)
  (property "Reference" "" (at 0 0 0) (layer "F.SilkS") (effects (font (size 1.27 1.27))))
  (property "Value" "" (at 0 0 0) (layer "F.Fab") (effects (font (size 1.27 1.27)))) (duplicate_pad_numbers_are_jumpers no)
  (pad "2" thru_hole oval (at 0 0) (size 1.8 1.8) (drill 0.7) (layers "*.Cu") (remove_unused_layers no)))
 (gr_line (start 0 0) (end 90.17 0) (stroke (width 0.15) (type default)) (layer "Edge.Cuts"))
 (gr_line (start 0 95.89) (end 0 0) (stroke (width 0.15) (type default)) (layer "Edge.Cuts"))
 (gr_line (start 90.17 0) (end 90.17 95.89) (stroke (width 0.15) (type default)) (layer "Edge.Cuts"))
 (gr_line (start 90.17 95.89) (end 0 95.89) (stroke (width 0.15) (type default)) (layer "Edge.Cuts"))
 (segment (start 22.085 42.195) (end 21.785 42.195) (width 0.6) (layer "F.Cu") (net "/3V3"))
 (segment (start 17.585 54.495) (end 15.885 56.195) (width 0.6) (layer "F.Cu") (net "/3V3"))
 (segment (start 21.785 42.195) (end 17.585 46.395) (width 0.6) (layer "F.Cu") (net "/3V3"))
 (segment (start 17.585 46.395) (end 17.585 54.495) (width 0.6) (layer "F.Cu") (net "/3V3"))
 (segment (start 33.585 42.195) (end 22.085 42.195) (width 0.6) (layer "B.Cu") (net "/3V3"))
 (segment (start 61.885 46.395) (end 57.185 46.395) (width 0.6) (layer "B.Cu") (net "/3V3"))
 (segment (start 45.285 34.495) (end 41.285 34.495) (width 0.6) (layer "B.Cu") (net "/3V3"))
 (segment (start 57.185 46.395) (end 45.285 34.495) (width 0.6) (layer "B.Cu") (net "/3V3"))
 (segment (start 41.285 34.495) (end 33.585 42.195) (width 0.6) (layer "B.Cu") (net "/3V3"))
 (segment (start 54.185 86.195) (end 63.085 86.195) (width 0.6) (layer "B.Cu") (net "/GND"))
 (segment (start 44.085 79.395) (end 47.385 79.395) (width 0.6) (layer "B.Cu") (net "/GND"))
 (segment (start 63.085 86.195) (end 63.385 85.895) (width 0.6) (layer "B.Cu") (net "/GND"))
 (segment (start 19.885 57.295) (end 19.885 46.595) (width 0.6) (layer "B.Cu") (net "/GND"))
 (segment (start 67.285 41.295) (end 61.885 41.295) (width 0.6) (layer "B.Cu") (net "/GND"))
 (segment (start 26.585 74.695) (end 26.585 71.995) (width 0.6) (layer "B.Cu") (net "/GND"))
 (segment (start 76.785 61.395) (end 76.785 61.295) (width 0.6) (layer "B.Cu") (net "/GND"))
 (segment (start 76.785 61.295) (end 78.485 59.595) (width 0.6) (layer "B.Cu") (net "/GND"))
 (segment (start 26.585 74.695) (end 31.285 79.395) (width 0.6) (layer "B.Cu") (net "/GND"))
 (segment (start 78.485 84.895) (end 78.485 63.095) (width 0.6) (layer "B.Cu") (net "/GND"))
 (segment (start 31.285 79.395) (end 44.085 79.395) (width 0.6) (layer "B.Cu") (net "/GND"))
 (segment (start 26.585 71.995) (end 15.885 61.295) (width 0.6) (layer "B.Cu") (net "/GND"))
 (segment (start 77.485 85.895) (end 78.485 84.895) (width 0.6) (layer "B.Cu") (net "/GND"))
 (segment (start 77.485 36.695) (end 71.885 36.695) (width 0.6) (layer "B.Cu") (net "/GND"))
 (segment (start 78.485 37.695) (end 77.485 36.695) (width 0.6) (layer "B.Cu") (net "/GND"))
 (segment (start 19.885 46.595) (end 21.685 44.795) (width 0.6) (layer "B.Cu") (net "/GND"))
 (segment (start 47.385 79.395) (end 54.185 86.195) (width 0.6) (layer "B.Cu") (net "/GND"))
 (segment (start 78.485 63.095) (end 76.785 61.395) (width 0.6) (layer "B.Cu") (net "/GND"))
 (segment (start 78.485 59.595) (end 78.485 37.695) (width 0.6) (layer "B.Cu") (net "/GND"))
 (segment (start 15.885 61.295) (end 19.885 57.295) (width 0.6) (layer "B.Cu") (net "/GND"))
 (segment (start 63.385 85.895) (end 77.485 85.895) (width 0.6) (layer "B.Cu") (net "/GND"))
 (segment (start 21.685 44.795) (end 22.085 44.795) (width 0.6) (layer "B.Cu") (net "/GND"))
 (segment (start 71.885 36.695) (end 67.285 41.295) (width 0.6) (layer "B.Cu") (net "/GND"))
 (segment (start 44.085 46.395) (end 43.585 46.395) (width 0.6) (layer "F.Cu") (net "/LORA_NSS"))
 (segment (start 21.085 68.895) (end 21.085 70.595) (width 0.6) (layer "F.Cu") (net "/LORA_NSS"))
 (segment (start 43.585 46.395) (end 21.085 68.895) (width 0.6) (layer "F.Cu") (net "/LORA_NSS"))
 (segment (start 21.085 71.295) (end 15.885 76.495) (width 0.6) (layer "B.Cu") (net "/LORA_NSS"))
 (segment (start 21.085 70.595) (end 21.085 71.295) (width 0.6) (layer "B.Cu") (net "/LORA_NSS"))
 (segment (start 17.585 69.895) (end 17.585 77.295) (width 0.6) (layer "F.Cu") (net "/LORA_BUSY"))
 (segment (start 17.585 77.295) (end 15.885 78.995) (width 0.6) (layer "F.Cu") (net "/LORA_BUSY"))
 (segment (start 43.685 43.795) (end 17.585 69.895) (width 0.6) (layer "F.Cu") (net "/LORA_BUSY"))
 (segment (start 44.085 43.795) (end 43.685 43.795) (width 0.6) (layer "F.Cu") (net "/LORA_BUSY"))
 (segment (start 43.685 84.095) (end 15.885 84.095) (width 0.6) (layer "B.Cu") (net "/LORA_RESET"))
 (segment (start 44.085 84.495) (end 43.685 84.095) (width 0.6) (layer "B.Cu") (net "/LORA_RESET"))
 (segment (start 59.085 84.595) (end 60.585 86.095) (width 0.6) (layer "F.Cu") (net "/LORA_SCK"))
 (segment (start 62.785 86.095) (end 63.085 86.095) (width 0.6) (layer "F.Cu") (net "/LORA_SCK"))
 (segment (start 63.085 86.095) (end 63.985 85.195) (width 0.6) (layer "F.Cu") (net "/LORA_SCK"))
 (segment (start 63.985 84.995) (end 64.085 84.895) (width 0.6) (layer "F.Cu") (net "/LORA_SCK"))
 (segment (start 60.885 86.095) (end 60.985 86.195) (width 0.6) (layer "F.Cu") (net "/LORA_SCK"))
 (segment (start 60.585 86.095) (end 60.885 86.095) (width 0.6) (layer "F.Cu") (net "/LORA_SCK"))
 (segment (start 44.585 69.195) (end 59.085 83.695) (width 0.6) (layer "F.Cu") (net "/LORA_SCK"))
 (segment (start 62.685 86.195) (end 62.785 86.095) (width 0.6) (layer "F.Cu") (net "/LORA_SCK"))
 (segment (start 64.085 61.295) (end 74.285 51.095) (width 0.6) (layer "F.Cu") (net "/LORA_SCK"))
 (segment (start 60.985 86.195) (end 62.685 86.195) (width 0.6) (layer "F.Cu") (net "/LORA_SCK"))
 (segment (start 63.985 85.195) (end 63.985 84.995) (width 0.6) (layer "F.Cu") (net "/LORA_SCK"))
 (segment (start 64.085 84.895) (end 64.085 61.295) (width 0.6) (layer "F.Cu") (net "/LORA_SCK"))
 (segment (start 44.085 69.195) (end 44.585 69.195) (width 0.6) (layer "F.Cu") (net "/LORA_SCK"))
 (segment (start 59.085 83.695) (end 59.085 84.595) (width 0.6) (layer "F.Cu") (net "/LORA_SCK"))
 (segment (start 65.985 86.295) (end 65.985 85.995) (width 0.6) (layer "F.Cu") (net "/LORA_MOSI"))
 (segment (start 65.685 86.595) (end 65.985 86.295) (width 0.6) (layer "F.Cu") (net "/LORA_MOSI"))
 (segment (start 65.985 85.995) (end 66.085 85.895) (width 0.6) (layer "F.Cu") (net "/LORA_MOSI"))
 (segment (start 71.585 62.095) (end 72.585 61.095) (width 0.6) (layer "F.Cu") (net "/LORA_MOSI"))
 (segment (start 64.285 88.195) (end 65.685 86.795) (width 0.6) (layer "F.Cu") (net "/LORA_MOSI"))
 (segment (start 55.085 83.995) (end 59.285 88.195) (width 0.6) (layer "F.Cu") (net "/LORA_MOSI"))
 (segment (start 71.585 69.395) (end 71.585 62.095) (width 0.6) (layer "F.Cu") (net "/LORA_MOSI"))
 (segment (start 66.085 74.895) (end 71.585 69.395) (width 0.6) (layer "F.Cu") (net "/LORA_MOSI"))
 (segment (start 59.285 88.195) (end 64.285 88.195) (width 0.6) (layer "F.Cu") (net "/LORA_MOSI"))
 (segment (start 72.585 61.095) (end 72.585 57.895) (width 0.6) (layer "F.Cu") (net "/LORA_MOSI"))
 (segment (start 66.085 85.895) (end 66.085 74.895) (width 0.6) (layer "F.Cu") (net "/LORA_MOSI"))
 (segment (start 72.585 57.895) (end 74.285 56.195) (width 0.6) (layer "F.Cu") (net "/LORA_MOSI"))
 (segment (start 65.685 86.795) (end 65.685 86.595) (width 0.6) (layer "F.Cu") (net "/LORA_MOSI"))
 (segment (start 44.085 71.795) (end 44.585 71.795) (width 0.6) (layer "B.Cu") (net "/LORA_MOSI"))
 (segment (start 55.085 82.295) (end 55.085 83.995) (width 0.6) (layer "B.Cu") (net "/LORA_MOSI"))
 (segment (start 44.585 71.795) (end 55.085 82.295) (width 0.6) (layer "B.Cu") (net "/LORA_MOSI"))
 (segment (start 59.985 86.895) (end 59.785 86.895) (width 0.6) (layer "F.Cu") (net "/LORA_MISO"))
 (segment (start 59.785 86.895) (end 56.685 83.795) (width 0.6) (layer "F.Cu") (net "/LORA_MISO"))
 (segment (start 60.185 87.095) (end 59.985 86.895) (width 0.6) (layer "F.Cu") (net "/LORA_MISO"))
 (segment (start 63.185 87.195) (end 60.485 87.195) (width 0.6) (layer "F.Cu") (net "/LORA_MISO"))
 (segment (start 64.885 85.795) (end 64.885 85.995) (width 0.6) (layer "F.Cu") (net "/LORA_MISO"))
 (segment (start 67.085 67.695) (end 67.085 72.095) (width 0.6) (layer "F.Cu") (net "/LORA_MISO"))
 (segment (start 65.085 74.095) (end 65.085 85.395) (width 0.6) (layer "F.Cu") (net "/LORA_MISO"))
 (segment (start 63.985 86.795) (end 63.685 87.095) (width 0.6) (layer "F.Cu") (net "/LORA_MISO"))
 (segment (start 64.985 85.695) (end 64.885 85.795) (width 0.6) (layer "F.Cu") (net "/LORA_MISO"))
 (segment (start 56.685 83.532258) (end 55.747742 82.595) (width 0.6) (layer "F.Cu") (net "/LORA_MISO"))
 (segment (start 64.085 86.795) (end 63.985 86.795) (width 0.6) (layer "F.Cu") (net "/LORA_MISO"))
 (segment (start 60.385 87.095) (end 60.185 87.095) (width 0.6) (layer "F.Cu") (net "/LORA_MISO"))
 (segment (start 65.085 85.395) (end 64.985 85.495) (width 0.6) (layer "F.Cu") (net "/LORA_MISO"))
 (segment (start 64.885 85.995) (end 64.085 86.795) (width 0.6) (layer "F.Cu") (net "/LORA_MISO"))
 (segment (start 55.747742 82.595) (end 55.485 82.595) (width 0.6) (layer "F.Cu") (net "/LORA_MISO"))
 (segment (start 67.085 72.095) (end 65.085 74.095) (width 0.6) (layer "F.Cu") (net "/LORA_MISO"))
 (segment (start 47.185 74.295) (end 44.085 74.295) (width 0.6) (layer "F.Cu") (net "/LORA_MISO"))
 (segment (start 63.685 87.095) (end 63.285 87.095) (width 0.6) (layer "F.Cu") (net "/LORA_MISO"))
 (segment (start 56.685 83.795) (end 56.685 83.532258) (width 0.6) (layer "F.Cu") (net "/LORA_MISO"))
 (segment (start 60.485 87.195) (end 60.385 87.095) (width 0.6) (layer "F.Cu") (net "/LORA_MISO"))
 (segment (start 64.985 85.495) (end 64.985 85.695) (width 0.6) (layer "F.Cu") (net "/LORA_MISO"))
 (segment (start 55.485 82.595) (end 47.185 74.295) (width 0.6) (layer "F.Cu") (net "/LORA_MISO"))
 (segment (start 63.285 87.095) (end 63.185 87.195) (width 0.6) (layer "F.Cu") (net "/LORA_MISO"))
 (segment (start 65.285 65.895) (end 65.285 62.595) (width 0.6) (layer "B.Cu") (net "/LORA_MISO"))
 (segment (start 67.085 67.695) (end 65.285 65.895) (width 0.6) (layer "B.Cu") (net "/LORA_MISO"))
 (segment (start 65.285 62.595) (end 74.285 53.595) (width 0.6) (layer "B.Cu") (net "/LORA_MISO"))
 (segment (start 73.485 85.795) (end 77.585 85.795) (width 0.6) (layer "F.Cu") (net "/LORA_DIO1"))
 (segment (start 77.585 85.795) (end 78.485 84.895) (width 0.6) (layer "F.Cu") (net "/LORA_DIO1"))
 (segment (start 78.485 67.995) (end 76.785 66.295) (width 0.6) (layer "F.Cu") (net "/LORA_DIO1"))
 (segment (start 78.485 84.895) (end 78.485 67.995) (width 0.6) (layer "F.Cu") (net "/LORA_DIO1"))
 (segment (start 71.735 84.045) (end 73.485 85.795) (width 0.6) (layer "F.Cu") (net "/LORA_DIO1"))
 (segment (start 64.085 76.395) (end 64.085 73.495) (width 0.6) (layer "B.Cu") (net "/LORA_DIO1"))
 (segment (start 64.085 73.495) (end 62.385 71.795) (width 0.6) (layer "B.Cu") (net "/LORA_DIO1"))
 (segment (start 71.735 84.045) (end 64.085 76.395) (width 0.6) (layer "B.Cu") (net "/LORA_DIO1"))
 (segment (start 62.385 71.795) (end 61.885 71.795) (width 0.6) (layer "B.Cu") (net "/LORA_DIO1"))
 (segment (start 68.085 85.895) (end 72.585 81.395) (width 0.6) (layer "F.Cu") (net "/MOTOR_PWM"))
 (segment (start 72.585 67.995) (end 74.285 66.295) (width 0.6) (layer "F.Cu") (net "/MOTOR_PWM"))
 (segment (start 72.585 81.395) (end 72.585 67.995) (width 0.6) (layer "F.Cu") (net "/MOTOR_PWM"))
 (segment (start 69.585 87.695) (end 68.085 86.195) (width 0.6) (layer "F.Cu") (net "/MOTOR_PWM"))
 (segment (start 24.085 74.995) (end 24.085 74.695) (width 0.6) (layer "F.Cu") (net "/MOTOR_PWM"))
 (segment (start 34.785 85.695) (end 24.085 74.995) (width 0.6) (layer "F.Cu") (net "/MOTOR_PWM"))
 (segment (start 39.585 85.695) (end 34.785 85.695) (width 0.6) (layer "F.Cu") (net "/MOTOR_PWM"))
 (segment (start 68.085 86.195) (end 68.085 85.895) (width 0.6) (layer "F.Cu") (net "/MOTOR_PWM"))
 (segment (start 67.585 87.695) (end 67.085 87.195) (width 0.6) (layer "B.Cu") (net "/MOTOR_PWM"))
 (segment (start 43.685 87.195) (end 42.185 85.695) (width 0.6) (layer "B.Cu") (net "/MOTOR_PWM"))
 (segment (start 67.085 87.195) (end 43.685 87.195) (width 0.6) (layer "B.Cu") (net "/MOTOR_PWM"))
 (segment (start 42.185 85.695) (end 39.585 85.695) (width 0.6) (layer "B.Cu") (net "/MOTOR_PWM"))
 (segment (start 69.585 87.695) (end 67.585 87.695) (width 0.6) (layer "B.Cu") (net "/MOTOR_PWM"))
 (segment (start 22.085 47.295) (end 22.985 47.295) (width 0.6) (layer "F.Cu") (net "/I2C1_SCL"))
 (segment (start 22.985 47.295) (end 36.785 33.495) (width 0.6) (layer "F.Cu") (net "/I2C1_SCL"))
 (segment (start 66.885 33.495) (end 74.285 40.895) (width 0.6) (layer "F.Cu") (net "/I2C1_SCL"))
 (segment (start 36.785 33.495) (end 66.885 33.495) (width 0.6) (layer "F.Cu") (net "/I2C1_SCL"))
 (segment (start 22.085 49.895) (end 27.485 49.895) (width 0.6) (layer "F.Cu") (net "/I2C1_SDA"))
 (segment (start 42.885 34.495) (end 65.285 34.495) (width 0.6) (layer "F.Cu") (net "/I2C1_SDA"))
 (segment (start 27.485 49.895) (end 42.885 34.495) (width 0.6) (layer "F.Cu") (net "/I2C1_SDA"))
 (segment (start 65.285 34.495) (end 74.285 43.495) (width 0.6) (layer "F.Cu") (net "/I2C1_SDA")))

